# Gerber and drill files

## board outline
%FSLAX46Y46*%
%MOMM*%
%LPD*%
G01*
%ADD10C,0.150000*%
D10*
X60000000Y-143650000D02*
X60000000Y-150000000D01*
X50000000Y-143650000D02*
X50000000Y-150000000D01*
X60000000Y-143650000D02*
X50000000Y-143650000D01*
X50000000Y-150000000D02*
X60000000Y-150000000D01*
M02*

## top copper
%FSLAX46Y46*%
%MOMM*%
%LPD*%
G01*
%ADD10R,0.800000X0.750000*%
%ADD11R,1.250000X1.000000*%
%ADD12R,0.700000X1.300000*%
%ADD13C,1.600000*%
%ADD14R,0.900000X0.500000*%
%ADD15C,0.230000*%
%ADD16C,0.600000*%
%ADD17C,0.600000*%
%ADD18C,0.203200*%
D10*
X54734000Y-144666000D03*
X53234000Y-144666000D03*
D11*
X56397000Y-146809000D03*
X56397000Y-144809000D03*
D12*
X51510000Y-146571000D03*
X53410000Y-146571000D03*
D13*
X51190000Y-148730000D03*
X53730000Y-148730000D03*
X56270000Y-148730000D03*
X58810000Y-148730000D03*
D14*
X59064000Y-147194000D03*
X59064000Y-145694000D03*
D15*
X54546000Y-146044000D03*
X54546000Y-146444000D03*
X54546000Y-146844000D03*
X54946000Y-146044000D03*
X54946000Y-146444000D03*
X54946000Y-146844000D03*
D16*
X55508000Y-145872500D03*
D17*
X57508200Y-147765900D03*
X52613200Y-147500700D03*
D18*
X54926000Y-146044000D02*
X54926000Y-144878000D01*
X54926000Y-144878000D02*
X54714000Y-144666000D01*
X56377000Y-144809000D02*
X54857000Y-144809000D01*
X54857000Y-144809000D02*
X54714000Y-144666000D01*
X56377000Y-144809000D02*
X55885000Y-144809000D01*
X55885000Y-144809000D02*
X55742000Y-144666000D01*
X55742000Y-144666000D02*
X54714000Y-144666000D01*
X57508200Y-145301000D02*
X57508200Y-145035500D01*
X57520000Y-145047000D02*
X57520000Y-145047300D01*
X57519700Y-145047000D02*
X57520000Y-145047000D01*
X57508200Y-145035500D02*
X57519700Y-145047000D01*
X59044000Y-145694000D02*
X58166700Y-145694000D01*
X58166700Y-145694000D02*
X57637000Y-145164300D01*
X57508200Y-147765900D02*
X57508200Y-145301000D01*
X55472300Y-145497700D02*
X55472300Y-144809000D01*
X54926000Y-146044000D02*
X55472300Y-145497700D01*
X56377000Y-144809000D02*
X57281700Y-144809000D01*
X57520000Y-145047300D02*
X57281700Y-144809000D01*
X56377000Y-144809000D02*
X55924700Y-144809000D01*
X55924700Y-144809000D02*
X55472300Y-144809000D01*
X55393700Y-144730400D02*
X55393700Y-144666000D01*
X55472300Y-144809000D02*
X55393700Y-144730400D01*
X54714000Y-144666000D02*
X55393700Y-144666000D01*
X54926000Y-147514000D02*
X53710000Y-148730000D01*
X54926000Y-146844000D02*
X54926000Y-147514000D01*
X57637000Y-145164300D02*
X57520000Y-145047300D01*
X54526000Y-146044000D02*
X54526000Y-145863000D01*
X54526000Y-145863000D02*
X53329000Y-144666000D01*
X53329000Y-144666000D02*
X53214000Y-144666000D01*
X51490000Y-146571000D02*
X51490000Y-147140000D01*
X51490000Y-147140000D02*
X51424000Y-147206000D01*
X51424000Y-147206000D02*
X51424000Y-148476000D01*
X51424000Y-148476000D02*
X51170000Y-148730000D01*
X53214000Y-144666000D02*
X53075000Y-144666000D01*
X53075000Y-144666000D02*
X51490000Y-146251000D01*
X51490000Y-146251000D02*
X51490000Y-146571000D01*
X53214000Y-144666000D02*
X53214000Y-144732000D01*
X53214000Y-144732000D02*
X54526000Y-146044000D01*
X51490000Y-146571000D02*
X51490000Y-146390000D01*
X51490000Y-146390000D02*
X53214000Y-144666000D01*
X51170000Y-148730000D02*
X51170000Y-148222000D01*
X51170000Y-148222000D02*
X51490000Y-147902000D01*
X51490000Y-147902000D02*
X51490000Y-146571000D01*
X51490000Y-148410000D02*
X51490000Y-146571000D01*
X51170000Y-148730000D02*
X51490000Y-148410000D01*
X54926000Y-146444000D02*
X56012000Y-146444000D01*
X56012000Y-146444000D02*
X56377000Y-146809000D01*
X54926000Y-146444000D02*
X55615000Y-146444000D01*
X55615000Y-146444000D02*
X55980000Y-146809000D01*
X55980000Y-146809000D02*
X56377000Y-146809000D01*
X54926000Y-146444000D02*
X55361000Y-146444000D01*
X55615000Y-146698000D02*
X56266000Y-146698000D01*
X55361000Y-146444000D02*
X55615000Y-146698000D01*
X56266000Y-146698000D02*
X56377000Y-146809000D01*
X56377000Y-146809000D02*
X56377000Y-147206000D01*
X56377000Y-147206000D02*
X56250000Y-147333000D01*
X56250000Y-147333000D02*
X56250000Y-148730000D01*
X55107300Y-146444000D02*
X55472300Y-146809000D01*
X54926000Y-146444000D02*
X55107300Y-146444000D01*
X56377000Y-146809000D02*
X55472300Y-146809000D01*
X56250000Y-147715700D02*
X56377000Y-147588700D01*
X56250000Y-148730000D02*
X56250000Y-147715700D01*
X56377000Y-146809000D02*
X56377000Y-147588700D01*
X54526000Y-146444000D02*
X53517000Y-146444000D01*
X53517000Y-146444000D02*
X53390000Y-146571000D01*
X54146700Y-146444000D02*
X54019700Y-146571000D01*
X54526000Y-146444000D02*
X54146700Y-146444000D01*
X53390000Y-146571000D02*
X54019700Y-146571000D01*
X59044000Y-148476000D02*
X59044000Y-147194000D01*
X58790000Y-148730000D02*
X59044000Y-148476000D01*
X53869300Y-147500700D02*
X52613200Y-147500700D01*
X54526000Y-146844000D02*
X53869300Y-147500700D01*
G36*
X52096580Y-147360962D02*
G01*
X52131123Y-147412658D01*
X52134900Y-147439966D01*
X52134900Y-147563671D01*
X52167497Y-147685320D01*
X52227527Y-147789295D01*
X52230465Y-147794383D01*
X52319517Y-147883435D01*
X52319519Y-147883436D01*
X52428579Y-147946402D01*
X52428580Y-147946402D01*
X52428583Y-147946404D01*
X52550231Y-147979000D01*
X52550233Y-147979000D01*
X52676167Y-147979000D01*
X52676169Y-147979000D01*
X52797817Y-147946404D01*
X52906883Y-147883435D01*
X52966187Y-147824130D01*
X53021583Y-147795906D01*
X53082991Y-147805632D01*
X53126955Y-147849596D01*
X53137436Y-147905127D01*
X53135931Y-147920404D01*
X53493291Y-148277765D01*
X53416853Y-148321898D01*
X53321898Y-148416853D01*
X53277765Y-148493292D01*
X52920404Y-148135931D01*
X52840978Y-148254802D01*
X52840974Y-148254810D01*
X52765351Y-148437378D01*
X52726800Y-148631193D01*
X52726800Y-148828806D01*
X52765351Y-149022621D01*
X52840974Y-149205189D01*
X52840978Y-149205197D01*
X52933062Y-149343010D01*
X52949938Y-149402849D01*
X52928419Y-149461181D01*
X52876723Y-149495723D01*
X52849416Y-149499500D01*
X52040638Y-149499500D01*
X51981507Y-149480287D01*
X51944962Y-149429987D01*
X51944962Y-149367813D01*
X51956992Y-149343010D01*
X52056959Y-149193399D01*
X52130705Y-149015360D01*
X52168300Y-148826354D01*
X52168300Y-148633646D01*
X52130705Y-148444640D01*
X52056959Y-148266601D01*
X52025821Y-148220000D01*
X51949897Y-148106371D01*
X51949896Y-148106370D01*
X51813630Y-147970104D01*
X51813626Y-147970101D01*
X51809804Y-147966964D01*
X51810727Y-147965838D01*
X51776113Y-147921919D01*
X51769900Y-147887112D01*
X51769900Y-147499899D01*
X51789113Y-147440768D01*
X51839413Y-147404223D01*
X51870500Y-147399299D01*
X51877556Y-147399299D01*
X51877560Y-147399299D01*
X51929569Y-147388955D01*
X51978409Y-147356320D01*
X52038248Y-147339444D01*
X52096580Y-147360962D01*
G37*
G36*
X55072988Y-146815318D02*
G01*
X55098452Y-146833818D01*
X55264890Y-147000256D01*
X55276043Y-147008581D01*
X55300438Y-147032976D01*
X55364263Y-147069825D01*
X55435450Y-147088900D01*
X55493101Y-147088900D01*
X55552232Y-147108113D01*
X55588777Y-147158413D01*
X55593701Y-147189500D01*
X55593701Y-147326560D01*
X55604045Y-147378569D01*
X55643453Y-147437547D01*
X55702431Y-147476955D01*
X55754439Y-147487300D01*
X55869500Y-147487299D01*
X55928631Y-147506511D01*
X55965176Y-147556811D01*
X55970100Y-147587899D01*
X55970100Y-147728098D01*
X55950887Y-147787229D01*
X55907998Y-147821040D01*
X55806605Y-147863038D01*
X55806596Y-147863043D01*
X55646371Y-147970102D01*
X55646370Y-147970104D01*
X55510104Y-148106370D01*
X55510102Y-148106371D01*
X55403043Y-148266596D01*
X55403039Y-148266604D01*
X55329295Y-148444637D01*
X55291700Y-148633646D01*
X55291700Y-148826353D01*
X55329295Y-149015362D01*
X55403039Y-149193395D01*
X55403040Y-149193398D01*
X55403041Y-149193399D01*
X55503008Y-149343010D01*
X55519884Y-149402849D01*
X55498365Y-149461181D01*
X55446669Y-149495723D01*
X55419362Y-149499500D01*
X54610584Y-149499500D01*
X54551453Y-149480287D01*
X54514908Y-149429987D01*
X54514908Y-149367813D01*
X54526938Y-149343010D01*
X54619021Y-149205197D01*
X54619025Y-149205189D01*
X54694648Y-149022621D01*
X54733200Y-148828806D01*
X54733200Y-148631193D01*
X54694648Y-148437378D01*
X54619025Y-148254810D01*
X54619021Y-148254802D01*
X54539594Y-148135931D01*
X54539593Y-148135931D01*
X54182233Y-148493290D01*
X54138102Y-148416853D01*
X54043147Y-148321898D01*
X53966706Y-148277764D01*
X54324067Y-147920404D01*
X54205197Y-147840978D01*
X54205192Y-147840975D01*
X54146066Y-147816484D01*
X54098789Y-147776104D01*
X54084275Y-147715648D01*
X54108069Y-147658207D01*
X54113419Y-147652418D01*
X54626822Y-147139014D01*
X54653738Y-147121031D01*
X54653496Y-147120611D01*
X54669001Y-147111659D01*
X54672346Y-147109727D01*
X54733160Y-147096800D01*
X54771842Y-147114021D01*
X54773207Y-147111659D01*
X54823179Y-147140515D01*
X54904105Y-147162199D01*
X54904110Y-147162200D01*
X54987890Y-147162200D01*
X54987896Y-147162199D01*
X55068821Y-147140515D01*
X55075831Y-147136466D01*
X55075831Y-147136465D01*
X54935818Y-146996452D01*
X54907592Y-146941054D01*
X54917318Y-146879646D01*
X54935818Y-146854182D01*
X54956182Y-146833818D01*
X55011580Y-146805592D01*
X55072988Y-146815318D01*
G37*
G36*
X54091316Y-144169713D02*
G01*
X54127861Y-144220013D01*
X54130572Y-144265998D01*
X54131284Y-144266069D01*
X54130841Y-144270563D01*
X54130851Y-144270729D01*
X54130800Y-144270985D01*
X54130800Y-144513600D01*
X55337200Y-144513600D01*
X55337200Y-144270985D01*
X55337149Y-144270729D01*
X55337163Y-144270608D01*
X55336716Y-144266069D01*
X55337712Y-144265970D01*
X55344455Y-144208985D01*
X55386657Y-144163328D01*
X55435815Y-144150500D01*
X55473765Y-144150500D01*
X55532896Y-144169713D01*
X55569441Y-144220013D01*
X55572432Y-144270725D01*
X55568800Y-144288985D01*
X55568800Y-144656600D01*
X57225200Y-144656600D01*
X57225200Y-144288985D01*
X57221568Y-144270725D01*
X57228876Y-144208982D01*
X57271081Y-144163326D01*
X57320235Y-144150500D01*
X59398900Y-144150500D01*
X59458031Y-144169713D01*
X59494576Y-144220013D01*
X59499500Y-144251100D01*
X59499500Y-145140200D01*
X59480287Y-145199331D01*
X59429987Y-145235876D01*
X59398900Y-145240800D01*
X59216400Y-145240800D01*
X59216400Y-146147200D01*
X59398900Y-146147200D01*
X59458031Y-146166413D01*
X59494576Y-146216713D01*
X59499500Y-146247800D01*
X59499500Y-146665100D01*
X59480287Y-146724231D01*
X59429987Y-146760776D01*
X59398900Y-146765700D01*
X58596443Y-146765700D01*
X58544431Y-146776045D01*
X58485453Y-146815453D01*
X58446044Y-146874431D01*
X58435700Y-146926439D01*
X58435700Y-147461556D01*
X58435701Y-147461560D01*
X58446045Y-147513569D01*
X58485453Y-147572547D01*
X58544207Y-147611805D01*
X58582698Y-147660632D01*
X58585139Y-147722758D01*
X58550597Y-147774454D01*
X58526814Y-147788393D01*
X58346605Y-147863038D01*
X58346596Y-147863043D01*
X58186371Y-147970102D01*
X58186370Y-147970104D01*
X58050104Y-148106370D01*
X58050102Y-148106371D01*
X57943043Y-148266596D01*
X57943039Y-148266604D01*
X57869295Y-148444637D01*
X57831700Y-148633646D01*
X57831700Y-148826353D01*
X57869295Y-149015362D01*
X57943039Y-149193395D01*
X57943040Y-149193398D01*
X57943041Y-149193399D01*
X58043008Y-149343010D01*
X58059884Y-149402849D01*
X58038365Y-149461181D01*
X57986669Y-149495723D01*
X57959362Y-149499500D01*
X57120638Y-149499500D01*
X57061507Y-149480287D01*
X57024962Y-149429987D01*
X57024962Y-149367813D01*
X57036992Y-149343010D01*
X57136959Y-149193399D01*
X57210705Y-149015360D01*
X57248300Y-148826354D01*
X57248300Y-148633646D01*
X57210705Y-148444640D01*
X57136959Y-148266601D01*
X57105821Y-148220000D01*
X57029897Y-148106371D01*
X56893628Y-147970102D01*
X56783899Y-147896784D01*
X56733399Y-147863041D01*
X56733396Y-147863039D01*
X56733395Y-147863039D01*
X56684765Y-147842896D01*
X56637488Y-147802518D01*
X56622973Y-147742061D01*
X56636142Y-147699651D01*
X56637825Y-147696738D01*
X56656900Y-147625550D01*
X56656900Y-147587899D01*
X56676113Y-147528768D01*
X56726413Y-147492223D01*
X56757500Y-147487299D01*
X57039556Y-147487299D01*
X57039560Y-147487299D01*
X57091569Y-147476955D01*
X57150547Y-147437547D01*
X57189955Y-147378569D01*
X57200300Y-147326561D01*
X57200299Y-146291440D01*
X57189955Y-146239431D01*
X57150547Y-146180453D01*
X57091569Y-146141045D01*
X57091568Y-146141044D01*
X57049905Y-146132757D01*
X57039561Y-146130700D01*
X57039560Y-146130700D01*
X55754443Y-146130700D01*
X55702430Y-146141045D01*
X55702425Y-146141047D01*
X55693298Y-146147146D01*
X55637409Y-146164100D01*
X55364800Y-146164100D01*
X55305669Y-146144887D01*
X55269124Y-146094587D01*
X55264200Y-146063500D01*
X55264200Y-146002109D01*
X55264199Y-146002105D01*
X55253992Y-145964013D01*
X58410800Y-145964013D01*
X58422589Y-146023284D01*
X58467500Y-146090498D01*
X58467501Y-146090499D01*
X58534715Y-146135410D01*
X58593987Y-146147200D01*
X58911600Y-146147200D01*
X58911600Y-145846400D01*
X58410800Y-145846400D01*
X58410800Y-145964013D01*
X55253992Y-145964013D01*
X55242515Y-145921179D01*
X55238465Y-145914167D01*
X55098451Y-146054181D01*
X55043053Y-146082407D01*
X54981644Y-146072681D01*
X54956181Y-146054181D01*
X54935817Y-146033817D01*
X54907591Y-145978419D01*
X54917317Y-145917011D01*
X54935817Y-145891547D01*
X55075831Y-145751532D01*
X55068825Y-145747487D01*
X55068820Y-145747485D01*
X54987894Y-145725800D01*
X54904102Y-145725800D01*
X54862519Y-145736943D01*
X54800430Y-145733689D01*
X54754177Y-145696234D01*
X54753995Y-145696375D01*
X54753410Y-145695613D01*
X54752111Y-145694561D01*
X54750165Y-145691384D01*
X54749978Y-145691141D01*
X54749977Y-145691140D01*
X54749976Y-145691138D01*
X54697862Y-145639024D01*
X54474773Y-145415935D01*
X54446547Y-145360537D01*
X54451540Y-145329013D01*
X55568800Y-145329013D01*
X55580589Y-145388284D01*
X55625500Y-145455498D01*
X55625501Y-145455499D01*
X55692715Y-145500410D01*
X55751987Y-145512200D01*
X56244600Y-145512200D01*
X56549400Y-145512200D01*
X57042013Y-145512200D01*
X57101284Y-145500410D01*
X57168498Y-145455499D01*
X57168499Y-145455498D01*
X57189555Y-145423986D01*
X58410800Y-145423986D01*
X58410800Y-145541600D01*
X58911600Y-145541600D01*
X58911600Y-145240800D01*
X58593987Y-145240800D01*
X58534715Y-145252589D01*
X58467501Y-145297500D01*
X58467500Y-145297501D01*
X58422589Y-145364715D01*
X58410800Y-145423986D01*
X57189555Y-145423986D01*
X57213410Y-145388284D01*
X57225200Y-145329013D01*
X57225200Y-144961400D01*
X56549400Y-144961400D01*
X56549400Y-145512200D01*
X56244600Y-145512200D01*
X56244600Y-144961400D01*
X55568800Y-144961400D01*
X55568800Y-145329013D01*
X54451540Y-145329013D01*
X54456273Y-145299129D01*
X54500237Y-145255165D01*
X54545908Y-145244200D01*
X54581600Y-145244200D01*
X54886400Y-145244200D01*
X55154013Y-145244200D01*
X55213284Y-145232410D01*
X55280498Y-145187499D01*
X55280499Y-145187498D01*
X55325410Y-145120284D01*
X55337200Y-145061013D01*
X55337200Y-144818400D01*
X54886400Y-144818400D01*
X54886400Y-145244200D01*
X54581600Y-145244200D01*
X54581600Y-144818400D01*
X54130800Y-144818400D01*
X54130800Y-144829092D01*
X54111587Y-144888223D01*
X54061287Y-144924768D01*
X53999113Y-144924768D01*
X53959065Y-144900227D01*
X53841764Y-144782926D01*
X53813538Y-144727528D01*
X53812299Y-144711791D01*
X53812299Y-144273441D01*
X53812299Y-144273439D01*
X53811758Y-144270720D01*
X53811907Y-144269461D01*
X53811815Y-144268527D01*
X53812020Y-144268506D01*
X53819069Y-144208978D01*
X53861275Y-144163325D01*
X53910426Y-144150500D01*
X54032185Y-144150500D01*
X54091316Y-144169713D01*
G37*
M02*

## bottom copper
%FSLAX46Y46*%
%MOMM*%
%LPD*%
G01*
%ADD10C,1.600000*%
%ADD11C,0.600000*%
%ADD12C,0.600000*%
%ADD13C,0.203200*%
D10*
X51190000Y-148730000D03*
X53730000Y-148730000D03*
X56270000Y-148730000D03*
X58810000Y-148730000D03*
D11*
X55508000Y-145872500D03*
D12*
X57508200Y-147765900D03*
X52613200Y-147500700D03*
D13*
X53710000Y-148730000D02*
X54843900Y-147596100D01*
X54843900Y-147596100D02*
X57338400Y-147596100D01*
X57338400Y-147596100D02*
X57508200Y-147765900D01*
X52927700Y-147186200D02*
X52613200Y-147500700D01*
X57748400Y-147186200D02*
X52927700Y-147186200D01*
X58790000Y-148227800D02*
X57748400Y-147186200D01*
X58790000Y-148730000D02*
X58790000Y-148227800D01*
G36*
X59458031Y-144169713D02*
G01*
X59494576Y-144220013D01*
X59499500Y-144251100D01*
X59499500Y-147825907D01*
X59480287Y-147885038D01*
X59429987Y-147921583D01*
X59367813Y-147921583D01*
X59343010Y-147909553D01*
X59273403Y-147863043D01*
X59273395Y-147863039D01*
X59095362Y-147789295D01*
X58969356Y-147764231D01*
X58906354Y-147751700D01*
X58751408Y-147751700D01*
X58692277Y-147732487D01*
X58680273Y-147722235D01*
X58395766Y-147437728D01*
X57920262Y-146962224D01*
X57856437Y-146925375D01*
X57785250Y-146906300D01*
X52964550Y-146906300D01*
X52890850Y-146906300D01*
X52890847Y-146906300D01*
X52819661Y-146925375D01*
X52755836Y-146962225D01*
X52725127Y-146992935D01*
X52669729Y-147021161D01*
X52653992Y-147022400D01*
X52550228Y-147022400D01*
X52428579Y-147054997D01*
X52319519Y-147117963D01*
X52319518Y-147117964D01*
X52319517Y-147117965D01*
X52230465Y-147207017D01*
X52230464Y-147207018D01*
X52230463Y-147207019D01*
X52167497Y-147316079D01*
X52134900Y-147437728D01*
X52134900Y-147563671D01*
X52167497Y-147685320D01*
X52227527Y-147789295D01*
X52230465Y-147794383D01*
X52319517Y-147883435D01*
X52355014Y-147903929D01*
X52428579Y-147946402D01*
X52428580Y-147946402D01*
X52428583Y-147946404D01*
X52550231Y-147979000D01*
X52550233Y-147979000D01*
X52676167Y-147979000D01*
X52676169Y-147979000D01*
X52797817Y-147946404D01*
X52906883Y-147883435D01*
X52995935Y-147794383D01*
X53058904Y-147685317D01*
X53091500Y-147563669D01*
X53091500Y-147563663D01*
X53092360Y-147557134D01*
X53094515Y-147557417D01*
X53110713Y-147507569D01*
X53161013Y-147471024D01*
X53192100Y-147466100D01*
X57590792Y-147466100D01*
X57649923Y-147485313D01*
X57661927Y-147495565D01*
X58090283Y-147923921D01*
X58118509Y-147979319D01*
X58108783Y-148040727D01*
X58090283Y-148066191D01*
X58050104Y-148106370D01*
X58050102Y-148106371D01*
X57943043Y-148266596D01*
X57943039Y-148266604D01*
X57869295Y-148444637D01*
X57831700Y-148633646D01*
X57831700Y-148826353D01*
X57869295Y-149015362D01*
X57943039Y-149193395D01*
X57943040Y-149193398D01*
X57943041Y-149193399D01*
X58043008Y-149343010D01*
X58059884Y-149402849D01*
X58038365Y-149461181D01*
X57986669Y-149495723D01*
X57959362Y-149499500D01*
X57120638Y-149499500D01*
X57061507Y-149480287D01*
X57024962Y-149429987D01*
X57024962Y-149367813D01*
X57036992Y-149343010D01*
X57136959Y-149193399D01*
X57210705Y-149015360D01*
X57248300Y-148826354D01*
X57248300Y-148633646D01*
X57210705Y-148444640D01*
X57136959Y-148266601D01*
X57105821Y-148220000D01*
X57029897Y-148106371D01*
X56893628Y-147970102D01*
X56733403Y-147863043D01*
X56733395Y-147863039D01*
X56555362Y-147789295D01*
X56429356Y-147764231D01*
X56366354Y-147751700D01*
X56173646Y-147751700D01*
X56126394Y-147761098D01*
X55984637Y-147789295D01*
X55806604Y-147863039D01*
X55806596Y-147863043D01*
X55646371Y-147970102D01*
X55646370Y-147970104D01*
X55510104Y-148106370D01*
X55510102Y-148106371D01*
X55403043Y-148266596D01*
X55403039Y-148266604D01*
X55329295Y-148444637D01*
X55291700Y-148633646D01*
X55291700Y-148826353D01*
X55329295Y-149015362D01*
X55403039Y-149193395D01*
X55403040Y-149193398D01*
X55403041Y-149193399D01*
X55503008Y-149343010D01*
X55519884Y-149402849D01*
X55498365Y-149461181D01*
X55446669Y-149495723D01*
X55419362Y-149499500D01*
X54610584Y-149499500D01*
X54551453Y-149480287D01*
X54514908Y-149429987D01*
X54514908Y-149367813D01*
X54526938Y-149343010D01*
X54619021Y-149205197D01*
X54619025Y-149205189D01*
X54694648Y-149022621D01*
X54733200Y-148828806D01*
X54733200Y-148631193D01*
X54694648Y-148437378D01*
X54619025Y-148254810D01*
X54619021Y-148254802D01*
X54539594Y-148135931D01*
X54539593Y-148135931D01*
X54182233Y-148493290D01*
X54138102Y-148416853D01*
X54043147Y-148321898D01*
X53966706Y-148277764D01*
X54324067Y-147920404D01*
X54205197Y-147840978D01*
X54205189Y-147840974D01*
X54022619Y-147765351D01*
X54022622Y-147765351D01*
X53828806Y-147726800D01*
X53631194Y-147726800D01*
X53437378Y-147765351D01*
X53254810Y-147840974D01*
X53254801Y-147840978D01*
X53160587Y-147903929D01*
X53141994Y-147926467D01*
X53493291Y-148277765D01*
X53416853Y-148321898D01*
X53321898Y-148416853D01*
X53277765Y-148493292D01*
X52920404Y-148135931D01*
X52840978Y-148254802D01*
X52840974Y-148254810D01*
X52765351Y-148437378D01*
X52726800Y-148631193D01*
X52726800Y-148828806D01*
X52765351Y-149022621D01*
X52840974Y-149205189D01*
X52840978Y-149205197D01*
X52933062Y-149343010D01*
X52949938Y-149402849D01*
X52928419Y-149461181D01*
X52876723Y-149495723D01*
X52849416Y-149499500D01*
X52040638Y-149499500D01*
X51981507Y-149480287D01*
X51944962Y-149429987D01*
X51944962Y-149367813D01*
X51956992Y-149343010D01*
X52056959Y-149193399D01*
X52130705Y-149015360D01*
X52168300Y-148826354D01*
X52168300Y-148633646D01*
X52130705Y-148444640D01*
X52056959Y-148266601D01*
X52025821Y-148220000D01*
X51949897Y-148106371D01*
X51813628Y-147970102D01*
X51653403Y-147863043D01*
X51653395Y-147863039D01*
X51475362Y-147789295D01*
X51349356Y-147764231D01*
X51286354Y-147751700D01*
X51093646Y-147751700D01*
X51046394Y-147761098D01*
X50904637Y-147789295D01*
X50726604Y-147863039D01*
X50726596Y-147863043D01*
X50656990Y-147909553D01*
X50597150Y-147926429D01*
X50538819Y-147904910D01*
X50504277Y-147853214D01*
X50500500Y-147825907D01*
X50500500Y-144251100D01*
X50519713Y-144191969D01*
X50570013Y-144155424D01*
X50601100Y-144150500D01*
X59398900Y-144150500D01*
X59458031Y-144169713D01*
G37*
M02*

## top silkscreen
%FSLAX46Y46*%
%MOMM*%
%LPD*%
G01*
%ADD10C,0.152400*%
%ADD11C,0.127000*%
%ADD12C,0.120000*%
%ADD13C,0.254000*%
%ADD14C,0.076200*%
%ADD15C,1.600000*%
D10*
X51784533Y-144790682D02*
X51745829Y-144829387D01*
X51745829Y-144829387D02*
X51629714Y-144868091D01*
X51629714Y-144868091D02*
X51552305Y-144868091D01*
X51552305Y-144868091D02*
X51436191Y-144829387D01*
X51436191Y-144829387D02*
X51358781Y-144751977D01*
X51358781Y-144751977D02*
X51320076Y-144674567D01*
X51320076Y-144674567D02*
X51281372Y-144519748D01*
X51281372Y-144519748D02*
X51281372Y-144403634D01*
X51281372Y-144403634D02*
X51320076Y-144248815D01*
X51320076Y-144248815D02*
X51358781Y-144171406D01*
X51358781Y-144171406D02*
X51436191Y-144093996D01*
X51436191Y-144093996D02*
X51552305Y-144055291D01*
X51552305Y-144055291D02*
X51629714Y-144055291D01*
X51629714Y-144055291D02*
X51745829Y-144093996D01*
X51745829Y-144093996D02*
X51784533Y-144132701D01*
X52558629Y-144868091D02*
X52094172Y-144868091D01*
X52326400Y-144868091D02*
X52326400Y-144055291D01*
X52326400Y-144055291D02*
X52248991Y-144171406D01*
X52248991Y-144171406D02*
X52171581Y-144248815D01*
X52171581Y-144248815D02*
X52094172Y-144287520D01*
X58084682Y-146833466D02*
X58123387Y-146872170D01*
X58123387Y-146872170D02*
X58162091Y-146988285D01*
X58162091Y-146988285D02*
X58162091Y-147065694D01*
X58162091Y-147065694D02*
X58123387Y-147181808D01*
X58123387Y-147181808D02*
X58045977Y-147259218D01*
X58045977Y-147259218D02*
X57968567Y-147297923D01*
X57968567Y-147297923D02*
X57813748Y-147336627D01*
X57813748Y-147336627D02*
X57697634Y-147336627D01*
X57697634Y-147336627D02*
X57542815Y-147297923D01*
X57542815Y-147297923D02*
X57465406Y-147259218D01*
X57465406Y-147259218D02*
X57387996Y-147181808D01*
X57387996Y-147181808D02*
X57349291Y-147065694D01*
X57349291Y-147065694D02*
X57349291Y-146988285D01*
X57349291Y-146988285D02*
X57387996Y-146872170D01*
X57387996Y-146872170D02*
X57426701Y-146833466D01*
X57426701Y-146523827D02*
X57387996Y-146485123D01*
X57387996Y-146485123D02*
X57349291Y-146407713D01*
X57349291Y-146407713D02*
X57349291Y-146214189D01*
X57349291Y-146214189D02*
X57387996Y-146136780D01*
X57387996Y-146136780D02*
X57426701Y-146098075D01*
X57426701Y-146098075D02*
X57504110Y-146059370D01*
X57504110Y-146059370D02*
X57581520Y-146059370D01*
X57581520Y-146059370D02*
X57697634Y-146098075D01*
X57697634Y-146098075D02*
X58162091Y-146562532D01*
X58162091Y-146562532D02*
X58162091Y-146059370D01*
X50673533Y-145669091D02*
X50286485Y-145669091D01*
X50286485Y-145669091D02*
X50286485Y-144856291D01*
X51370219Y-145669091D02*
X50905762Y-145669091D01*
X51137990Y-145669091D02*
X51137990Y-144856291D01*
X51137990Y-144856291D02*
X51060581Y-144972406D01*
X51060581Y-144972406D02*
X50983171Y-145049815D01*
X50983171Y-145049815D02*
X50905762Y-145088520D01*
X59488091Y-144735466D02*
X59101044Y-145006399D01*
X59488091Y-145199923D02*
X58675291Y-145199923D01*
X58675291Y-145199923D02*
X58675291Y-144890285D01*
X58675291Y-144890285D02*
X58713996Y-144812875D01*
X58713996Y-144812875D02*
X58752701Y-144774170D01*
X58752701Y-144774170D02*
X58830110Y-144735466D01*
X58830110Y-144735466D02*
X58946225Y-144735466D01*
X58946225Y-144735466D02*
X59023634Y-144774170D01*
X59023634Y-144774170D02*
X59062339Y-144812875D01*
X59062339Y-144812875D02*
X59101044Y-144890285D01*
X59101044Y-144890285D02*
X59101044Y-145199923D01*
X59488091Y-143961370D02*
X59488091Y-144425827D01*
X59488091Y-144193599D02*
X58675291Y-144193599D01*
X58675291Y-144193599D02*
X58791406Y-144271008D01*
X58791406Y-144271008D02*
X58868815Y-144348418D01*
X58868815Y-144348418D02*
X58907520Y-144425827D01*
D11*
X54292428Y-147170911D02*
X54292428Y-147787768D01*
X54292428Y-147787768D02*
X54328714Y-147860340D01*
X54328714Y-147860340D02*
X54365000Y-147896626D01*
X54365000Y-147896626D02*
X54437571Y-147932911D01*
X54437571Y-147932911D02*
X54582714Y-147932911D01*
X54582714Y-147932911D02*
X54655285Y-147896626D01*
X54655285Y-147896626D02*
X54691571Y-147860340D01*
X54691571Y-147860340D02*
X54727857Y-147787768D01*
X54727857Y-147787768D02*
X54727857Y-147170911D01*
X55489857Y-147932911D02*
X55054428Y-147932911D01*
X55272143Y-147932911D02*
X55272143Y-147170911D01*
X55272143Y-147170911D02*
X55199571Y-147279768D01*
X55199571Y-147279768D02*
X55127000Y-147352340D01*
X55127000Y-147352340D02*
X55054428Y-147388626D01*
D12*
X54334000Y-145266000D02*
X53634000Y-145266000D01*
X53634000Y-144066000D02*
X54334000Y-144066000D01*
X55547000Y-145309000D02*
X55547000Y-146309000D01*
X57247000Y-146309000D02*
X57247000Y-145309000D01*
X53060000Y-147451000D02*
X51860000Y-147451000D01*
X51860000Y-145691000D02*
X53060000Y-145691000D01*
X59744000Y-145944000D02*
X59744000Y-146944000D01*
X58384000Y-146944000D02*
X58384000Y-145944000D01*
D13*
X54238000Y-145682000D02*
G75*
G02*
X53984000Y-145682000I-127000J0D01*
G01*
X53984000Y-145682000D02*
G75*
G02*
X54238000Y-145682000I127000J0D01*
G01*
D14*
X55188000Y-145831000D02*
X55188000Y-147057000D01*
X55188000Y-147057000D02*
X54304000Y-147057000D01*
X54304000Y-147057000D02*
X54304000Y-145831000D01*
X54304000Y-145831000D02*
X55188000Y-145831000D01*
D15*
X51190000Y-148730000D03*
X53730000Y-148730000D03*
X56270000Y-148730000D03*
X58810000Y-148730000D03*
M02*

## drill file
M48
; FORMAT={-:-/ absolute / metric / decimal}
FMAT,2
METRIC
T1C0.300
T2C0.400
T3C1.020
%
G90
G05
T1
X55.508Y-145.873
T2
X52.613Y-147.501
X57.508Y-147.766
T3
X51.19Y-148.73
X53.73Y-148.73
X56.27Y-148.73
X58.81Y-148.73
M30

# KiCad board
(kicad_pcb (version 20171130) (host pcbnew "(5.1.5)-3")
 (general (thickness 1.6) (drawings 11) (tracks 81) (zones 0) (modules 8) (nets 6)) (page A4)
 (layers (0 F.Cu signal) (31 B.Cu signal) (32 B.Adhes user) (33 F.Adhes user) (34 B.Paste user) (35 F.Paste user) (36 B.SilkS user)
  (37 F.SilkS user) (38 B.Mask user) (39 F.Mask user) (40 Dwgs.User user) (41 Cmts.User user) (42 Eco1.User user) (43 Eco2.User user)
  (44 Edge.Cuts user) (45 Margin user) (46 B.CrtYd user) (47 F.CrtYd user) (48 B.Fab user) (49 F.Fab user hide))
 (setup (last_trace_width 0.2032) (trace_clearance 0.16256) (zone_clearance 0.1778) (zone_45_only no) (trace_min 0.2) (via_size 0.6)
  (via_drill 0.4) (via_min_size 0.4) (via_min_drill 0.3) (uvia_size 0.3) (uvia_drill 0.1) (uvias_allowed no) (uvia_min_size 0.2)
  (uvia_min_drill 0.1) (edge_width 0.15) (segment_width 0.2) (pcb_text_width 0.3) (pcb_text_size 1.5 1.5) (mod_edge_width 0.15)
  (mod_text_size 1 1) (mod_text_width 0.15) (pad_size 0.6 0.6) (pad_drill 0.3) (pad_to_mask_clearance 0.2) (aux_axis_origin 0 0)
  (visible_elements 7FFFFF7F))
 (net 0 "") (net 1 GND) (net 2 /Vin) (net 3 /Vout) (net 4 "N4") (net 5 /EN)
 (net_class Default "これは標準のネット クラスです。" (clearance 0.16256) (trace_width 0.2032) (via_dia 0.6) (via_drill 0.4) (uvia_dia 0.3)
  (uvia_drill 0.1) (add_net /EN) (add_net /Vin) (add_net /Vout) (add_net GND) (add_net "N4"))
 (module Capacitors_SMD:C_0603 (layer F.Cu) (at 53.984 144.666)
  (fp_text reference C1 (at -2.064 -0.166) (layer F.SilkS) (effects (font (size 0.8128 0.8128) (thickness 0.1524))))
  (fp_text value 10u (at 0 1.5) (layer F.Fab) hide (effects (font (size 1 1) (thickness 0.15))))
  (fp_line (start 0.35 0.6) (end -0.35 0.6) (layer F.SilkS) (width 0.12))
  (fp_line (start -0.35 -0.6) (end 0.35 -0.6) (layer F.SilkS) (width 0.12))
  (pad 2 smd rect (at 0.75 0) (size 0.8 0.75) (layers F.Cu F.Paste F.Mask) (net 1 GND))
  (pad 1 smd rect (at -0.75 0) (size 0.8 0.75) (layers F.Cu F.Paste F.Mask) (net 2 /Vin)))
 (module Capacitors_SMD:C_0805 (layer F.Cu) (at 56.397 145.809 90)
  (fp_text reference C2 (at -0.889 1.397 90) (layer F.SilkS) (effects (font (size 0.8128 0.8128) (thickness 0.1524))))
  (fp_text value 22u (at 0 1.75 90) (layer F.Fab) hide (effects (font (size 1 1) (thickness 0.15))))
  (fp_line (start 0.5 -0.85) (end -0.5 -0.85) (layer F.SilkS) (width 0.12))
  (fp_line (start -0.5 0.85) (end 0.5 0.85) (layer F.SilkS) (width 0.12))
  (pad 1 smd rect (at -1 0 90) (size 1 1.25) (layers F.Cu F.Paste F.Mask) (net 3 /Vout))
  (pad 2 smd rect (at 1 0 90) (size 1 1.25) (layers F.Cu F.Paste F.Mask) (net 1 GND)))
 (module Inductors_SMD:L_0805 (layer F.Cu) (at 52.46 146.571)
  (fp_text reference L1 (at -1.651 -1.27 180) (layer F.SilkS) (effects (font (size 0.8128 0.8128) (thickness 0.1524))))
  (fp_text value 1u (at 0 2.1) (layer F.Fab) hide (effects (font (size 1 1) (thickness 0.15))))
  (fp_line (start 0.6 0.88) (end -0.6 0.88) (layer F.SilkS) (width 0.12))
  (fp_line (start -0.6 -0.88) (end 0.6 -0.88) (layer F.SilkS) (width 0.12))
  (pad 1 smd rect (at -0.95 0) (size 0.7 1.3) (layers F.Cu F.Paste F.Mask) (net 2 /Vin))
  (pad 2 smd rect (at 0.95 0) (size 0.7 1.3) (layers F.Cu F.Paste F.Mask) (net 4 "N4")))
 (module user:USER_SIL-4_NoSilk (layer F.Cu) (at 55 148.73)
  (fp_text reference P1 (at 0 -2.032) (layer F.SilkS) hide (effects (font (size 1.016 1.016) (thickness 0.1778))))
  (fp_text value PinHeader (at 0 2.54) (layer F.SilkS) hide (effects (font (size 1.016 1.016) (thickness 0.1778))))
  (pad 1 thru_hole circle (at -3.81 0) (size 1.6 1.6) (drill 1.02) (layers *.Cu *.Mask F.SilkS) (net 2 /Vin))
  (pad 2 thru_hole circle (at -1.27 0) (size 1.6 1.6) (drill 1.02) (layers *.Cu *.Mask F.SilkS) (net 1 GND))
  (pad 3 thru_hole circle (at 1.27 0) (size 1.6 1.6) (drill 1.02) (layers *.Cu *.Mask F.SilkS) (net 3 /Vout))
  (pad 4 thru_hole circle (at 3.81 0) (size 1.6 1.6) (drill 1.02) (layers *.Cu *.Mask F.SilkS) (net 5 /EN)))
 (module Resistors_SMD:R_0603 (layer F.Cu) (at 59.064 146.444 90)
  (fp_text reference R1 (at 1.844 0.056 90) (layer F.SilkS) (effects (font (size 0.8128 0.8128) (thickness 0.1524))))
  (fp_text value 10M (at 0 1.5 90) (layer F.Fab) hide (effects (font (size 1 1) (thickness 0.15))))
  (fp_line (start 0.5 0.68) (end -0.5 0.68) (layer F.SilkS) (width 0.12))
  (fp_line (start -0.5 -0.68) (end 0.5 -0.68) (layer F.SilkS) (width 0.12))
  (pad 1 smd rect (at -0.75 0 90) (size 0.5 0.9) (layers F.Cu F.Paste F.Mask) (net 5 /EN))
  (pad 2 smd rect (at 0.75 0 90) (size 0.5 0.9) (layers F.Cu F.Paste F.Mask) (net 1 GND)))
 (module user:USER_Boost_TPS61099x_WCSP (layer F.Cu) (at 54.746 146.444)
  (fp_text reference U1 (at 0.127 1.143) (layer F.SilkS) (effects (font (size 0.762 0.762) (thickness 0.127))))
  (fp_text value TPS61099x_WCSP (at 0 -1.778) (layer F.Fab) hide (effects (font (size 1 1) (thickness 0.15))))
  (fp_circle (center -0.635 -0.762) (end -0.508 -0.762) (layer F.SilkS) (width 0.254))
  (fp_line (start 0.442 -0.613) (end 0.442 0.613) (layer F.SilkS) (width 0.0762))
  (fp_line (start 0.442 0.613) (end -0.442 0.613) (layer F.SilkS) (width 0.0762))
  (fp_line (start -0.442 0.613) (end -0.442 -0.613) (layer F.SilkS) (width 0.0762))
  (fp_line (start -0.442 -0.613) (end 0.442 -0.613) (layer F.SilkS) (width 0.0762))
  (pad A1 smd circle (at -0.2 -0.4) (size 0.23 0.23) (layers F.Cu F.Paste F.Mask) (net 2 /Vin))
  (pad B1 smd circle (at -0.2 0) (size 0.23 0.23) (layers F.Cu F.Paste F.Mask) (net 4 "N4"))
  (pad C1 smd circle (at -0.2 0.4) (size 0.23 0.23) (layers F.Cu F.Paste F.Mask) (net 5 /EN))
  (pad A2 smd circle (at 0.2 -0.4) (size 0.23 0.23) (layers F.Cu F.Paste F.Mask) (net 1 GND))
  (pad B2 smd circle (at 0.2 0) (size 0.23 0.23) (layers F.Cu F.Paste F.Mask) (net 3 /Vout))
  (pad C2 smd circle (at 0.2 0.4) (size 0.23 0.23) (layers F.Cu F.Paste F.Mask) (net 1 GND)))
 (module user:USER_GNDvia (layer F.Cu) (at 61.33 145.555)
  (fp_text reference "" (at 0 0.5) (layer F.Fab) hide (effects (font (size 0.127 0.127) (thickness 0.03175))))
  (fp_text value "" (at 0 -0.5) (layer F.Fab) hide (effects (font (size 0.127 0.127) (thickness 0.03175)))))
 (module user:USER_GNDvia (layer F.Cu) (at 55.508 145.8725)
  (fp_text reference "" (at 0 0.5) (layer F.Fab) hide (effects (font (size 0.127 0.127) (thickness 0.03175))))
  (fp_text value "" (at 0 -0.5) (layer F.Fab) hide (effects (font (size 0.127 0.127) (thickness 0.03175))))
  (pad "" thru_hole circle (at 0 0) (size 0.6 0.6) (drill 0.3) (layers *.Cu) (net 1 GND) (solder_mask_margin -0.000001)
   (clearance -0.000001) (zone_connect 2)))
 (gr_line (start 60 143.65) (end 60 150) (angle 90) (layer Edge.Cuts) (width 0.15))
 (gr_line (start 50 143.65) (end 50 150) (angle 90) (layer Edge.Cuts) (width 0.15))
 (gr_line (start 60 143.65) (end 50 143.65) (angle 90) (layer Edge.Cuts) (width 0.15))
 (gr_line (start 50 150) (end 60 150) (angle 90) (layer Edge.Cuts) (width 0.15))
 (segment (start 54.926 146.044) (end 54.926 144.878) (width 0.2032) (layer F.Cu) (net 1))
 (segment (start 54.926 144.878) (end 54.714 144.666) (width 0.2032) (layer F.Cu) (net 1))
 (segment (start 56.377 144.809) (end 54.857 144.809) (width 0.2032) (layer F.Cu) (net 1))
 (segment (start 54.857 144.809) (end 54.714 144.666) (width 0.2032) (layer F.Cu) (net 1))
 (segment (start 56.377 144.809) (end 55.885 144.809) (width 0.2032) (layer F.Cu) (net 1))
 (segment (start 55.885 144.809) (end 55.742 144.666) (width 0.2032) (layer F.Cu) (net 1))
 (segment (start 55.742 144.666) (end 54.714 144.666) (width 0.2032) (layer F.Cu) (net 1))
 (segment (start 57.5082 145.301) (end 57.5082 145.0355) (width 0.2032) (layer F.Cu) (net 1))
 (segment (start 57.52 145.047) (end 57.52 145.0473) (width 0.2032) (layer F.Cu) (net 1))
 (segment (start 57.5197 145.047) (end 57.52 145.047) (width 0.2032) (layer F.Cu) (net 1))
 (segment (start 57.5082 145.0355) (end 57.5197 145.047) (width 0.2032) (layer F.Cu) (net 1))
 (segment (start 59.044 145.694) (end 58.1667 145.694) (width 0.2032) (layer F.Cu) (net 1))
 (segment (start 58.1667 145.694) (end 57.637 145.1643) (width 0.2032) (layer F.Cu) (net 1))
 (via (at 57.5082 147.7659) (size 0.6) (layers F.Cu B.Cu) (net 1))
 (segment (start 57.5082 147.7659) (end 57.5082 145.301) (width 0.2032) (layer F.Cu) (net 1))
 (segment (start 53.71 148.73) (end 54.8439 147.5961) (width 0.2032) (layer B.Cu) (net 1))
 (segment (start 54.8439 147.5961) (end 57.3384 147.5961) (width 0.2032) (layer B.Cu) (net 1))
 (segment (start 57.3384 147.5961) (end 57.5082 147.7659) (width 0.2032) (layer B.Cu) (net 1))
 (segment (start 55.4723 145.4977) (end 55.4723 144.809) (width 0.2032) (layer F.Cu) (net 1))
 (segment (start 54.926 146.044) (end 55.4723 145.4977) (width 0.2032) (layer F.Cu) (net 1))
 (segment (start 56.377 144.809) (end 57.2817 144.809) (width 0.2032) (layer F.Cu) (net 1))
 (segment (start 57.52 145.0473) (end 57.2817 144.809) (width 0.2032) (layer F.Cu) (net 1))
 (segment (start 56.377 144.809) (end 55.9247 144.809) (width 0.2032) (layer F.Cu) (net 1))
 (segment (start 55.9247 144.809) (end 55.4723 144.809) (width 0.2032) (layer F.Cu) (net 1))
 (segment (start 55.3937 144.7304) (end 55.3937 144.666) (width 0.2032) (layer F.Cu) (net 1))
 (segment (start 55.4723 144.809) (end 55.3937 144.7304) (width 0.2032) (layer F.Cu) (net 1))
 (segment (start 54.714 144.666) (end 55.3937 144.666) (width 0.2032) (layer F.Cu) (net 1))
 (segment (start 54.926 147.514) (end 53.71 148.73) (width 0.2032) (layer F.Cu) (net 1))
 (segment (start 54.926 146.844) (end 54.926 147.514) (width 0.2032) (layer F.Cu) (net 1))
 (segment (start 57.637 145.1643) (end 57.52 145.0473) (width 0.2032) (layer F.Cu) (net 1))
 (segment (start 54.526 146.044) (end 54.526 145.863) (width 0.2032) (layer F.Cu) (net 2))
 (segment (start 54.526 145.863) (end 53.329 144.666) (width 0.2032) (layer F.Cu) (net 2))
 (segment (start 53.329 144.666) (end 53.214 144.666) (width 0.2032) (layer F.Cu) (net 2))
 (segment (start 51.49 146.571) (end 51.49 147.14) (width 0.2032) (layer F.Cu) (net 2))
 (segment (start 51.49 147.14) (end 51.424 147.206) (width 0.2032) (layer F.Cu) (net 2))
 (segment (start 51.424 147.206) (end 51.424 148.476) (width 0.2032) (layer F.Cu) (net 2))
 (segment (start 51.424 148.476) (end 51.17 148.73) (width 0.2032) (layer F.Cu) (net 2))
 (segment (start 53.214 144.666) (end 53.075 144.666) (width 0.2032) (layer F.Cu) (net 2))
 (segment (start 53.075 144.666) (end 51.49 146.251) (width 0.2032) (layer F.Cu) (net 2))
 (segment (start 51.49 146.251) (end 51.49 146.571) (width 0.2032) (layer F.Cu) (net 2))
 (segment (start 53.214 144.666) (end 53.214 144.732) (width 0.2032) (layer F.Cu) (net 2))
 (segment (start 53.214 144.732) (end 54.526 146.044) (width 0.2032) (layer F.Cu) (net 2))
 (segment (start 51.49 146.571) (end 51.49 146.39) (width 0.2032) (layer F.Cu) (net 2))
 (segment (start 51.49 146.39) (end 53.214 144.666) (width 0.2032) (layer F.Cu) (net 2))
 (segment (start 51.17 148.73) (end 51.17 148.222) (width 0.2032) (layer F.Cu) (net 2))
 (segment (start 51.17 148.222) (end 51.49 147.902) (width 0.2032) (layer F.Cu) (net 2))
 (segment (start 51.49 147.902) (end 51.49 146.571) (width 0.2032) (layer F.Cu) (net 2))
 (segment (start 51.49 148.41) (end 51.49 146.571) (width 0.2032) (layer F.Cu) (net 2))
 (segment (start 51.17 148.73) (end 51.49 148.41) (width 0.2032) (layer F.Cu) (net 2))
 (segment (start 54.926 146.444) (end 56.012 146.444) (width 0.2032) (layer F.Cu) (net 3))
 (segment (start 56.012 146.444) (end 56.377 146.809) (width 0.2032) (layer F.Cu) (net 3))
 (segment (start 54.926 146.444) (end 55.615 146.444) (width 0.2032) (layer F.Cu) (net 3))
 (segment (start 55.615 146.444) (end 55.98 146.809) (width 0.2032) (layer F.Cu) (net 3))
 (segment (start 55.98 146.809) (end 56.377 146.809) (width 0.2032) (layer F.Cu) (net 3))
 (segment (start 54.926 146.444) (end 55.361 146.444) (width 0.2032) (layer F.Cu) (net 3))
 (segment (start 55.615 146.698) (end 56.266 146.698) (width 0.2032) (layer F.Cu) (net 3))
 (segment (start 55.361 146.444) (end 55.615 146.698) (width 0.2032) (layer F.Cu) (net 3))
 (segment (start 56.266 146.698) (end 56.377 146.809) (width 0.2032) (layer F.Cu) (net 3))
 (segment (start 56.377 146.809) (end 56.377 147.206) (width 0.2032) (layer F.Cu) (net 3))
 (segment (start 56.377 147.206) (end 56.25 147.333) (width 0.2032) (layer F.Cu) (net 3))
 (segment (start 56.25 147.333) (end 56.25 148.73) (width 0.2032) (layer F.Cu) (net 3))
 (segment (start 55.1073 146.444) (end 55.4723 146.809) (width 0.2032) (layer F.Cu) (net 3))
 (segment (start 54.926 146.444) (end 55.1073 146.444) (width 0.2032) (layer F.Cu) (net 3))
 (segment (start 56.377 146.809) (end 55.4723 146.809) (width 0.2032) (layer F.Cu) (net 3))
 (segment (start 56.25 147.7157) (end 56.377 147.5887) (width 0.2032) (layer F.Cu) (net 3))
 (segment (start 56.25 148.73) (end 56.25 147.7157) (width 0.2032) (layer F.Cu) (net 3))
 (segment (start 56.377 146.809) (end 56.377 147.5887) (width 0.2032) (layer F.Cu) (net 3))
 (segment (start 54.526 146.444) (end 53.517 146.444) (width 0.2032) (layer F.Cu) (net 4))
 (segment (start 53.517 146.444) (end 53.39 146.571) (width 0.2032) (layer F.Cu) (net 4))
 (segment (start 54.1467 146.444) (end 54.0197 146.571) (width 0.2032) (layer F.Cu) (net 4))
 (segment (start 54.526 146.444) (end 54.1467 146.444) (width 0.2032) (layer F.Cu) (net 4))
 (segment (start 53.39 146.571) (end 54.0197 146.571) (width 0.2032) (layer F.Cu) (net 4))
 (via (at 52.6132 147.5007) (size 0.6) (layers F.Cu B.Cu) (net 5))
 (segment (start 59.044 148.476) (end 59.044 147.194) (width 0.2032) (layer F.Cu) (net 5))
 (segment (start 58.79 148.73) (end 59.044 148.476) (width 0.2032) (layer F.Cu) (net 5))
 (segment (start 52.9277 147.1862) (end 52.6132 147.5007) (width 0.2032) (layer B.Cu) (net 5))
 (segment (start 57.7484 147.1862) (end 52.9277 147.1862) (width 0.2032) (layer B.Cu) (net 5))
 (segment (start 58.79 148.2278) (end 57.7484 147.1862) (width 0.2032) (layer B.Cu) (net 5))
 (segment (start 58.79 148.73) (end 58.79 148.2278) (width 0.2032) (layer B.Cu) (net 5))
 (segment (start 53.8693 147.5007) (end 52.6132 147.5007) (width 0.2032) (layer F.Cu) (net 5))
 (segment (start 54.526 146.844) (end 53.8693 147.5007) (width 0.2032) (layer F.Cu) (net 5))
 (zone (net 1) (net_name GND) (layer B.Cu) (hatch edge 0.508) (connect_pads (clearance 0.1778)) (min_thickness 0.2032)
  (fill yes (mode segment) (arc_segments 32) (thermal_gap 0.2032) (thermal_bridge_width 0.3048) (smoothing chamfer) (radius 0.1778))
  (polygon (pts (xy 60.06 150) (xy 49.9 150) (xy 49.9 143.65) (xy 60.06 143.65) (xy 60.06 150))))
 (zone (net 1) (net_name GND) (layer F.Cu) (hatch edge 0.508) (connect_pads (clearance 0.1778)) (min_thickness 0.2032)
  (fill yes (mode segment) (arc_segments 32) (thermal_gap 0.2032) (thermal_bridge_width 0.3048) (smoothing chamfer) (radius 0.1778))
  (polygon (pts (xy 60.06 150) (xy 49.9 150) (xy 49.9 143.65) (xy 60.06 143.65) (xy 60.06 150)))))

